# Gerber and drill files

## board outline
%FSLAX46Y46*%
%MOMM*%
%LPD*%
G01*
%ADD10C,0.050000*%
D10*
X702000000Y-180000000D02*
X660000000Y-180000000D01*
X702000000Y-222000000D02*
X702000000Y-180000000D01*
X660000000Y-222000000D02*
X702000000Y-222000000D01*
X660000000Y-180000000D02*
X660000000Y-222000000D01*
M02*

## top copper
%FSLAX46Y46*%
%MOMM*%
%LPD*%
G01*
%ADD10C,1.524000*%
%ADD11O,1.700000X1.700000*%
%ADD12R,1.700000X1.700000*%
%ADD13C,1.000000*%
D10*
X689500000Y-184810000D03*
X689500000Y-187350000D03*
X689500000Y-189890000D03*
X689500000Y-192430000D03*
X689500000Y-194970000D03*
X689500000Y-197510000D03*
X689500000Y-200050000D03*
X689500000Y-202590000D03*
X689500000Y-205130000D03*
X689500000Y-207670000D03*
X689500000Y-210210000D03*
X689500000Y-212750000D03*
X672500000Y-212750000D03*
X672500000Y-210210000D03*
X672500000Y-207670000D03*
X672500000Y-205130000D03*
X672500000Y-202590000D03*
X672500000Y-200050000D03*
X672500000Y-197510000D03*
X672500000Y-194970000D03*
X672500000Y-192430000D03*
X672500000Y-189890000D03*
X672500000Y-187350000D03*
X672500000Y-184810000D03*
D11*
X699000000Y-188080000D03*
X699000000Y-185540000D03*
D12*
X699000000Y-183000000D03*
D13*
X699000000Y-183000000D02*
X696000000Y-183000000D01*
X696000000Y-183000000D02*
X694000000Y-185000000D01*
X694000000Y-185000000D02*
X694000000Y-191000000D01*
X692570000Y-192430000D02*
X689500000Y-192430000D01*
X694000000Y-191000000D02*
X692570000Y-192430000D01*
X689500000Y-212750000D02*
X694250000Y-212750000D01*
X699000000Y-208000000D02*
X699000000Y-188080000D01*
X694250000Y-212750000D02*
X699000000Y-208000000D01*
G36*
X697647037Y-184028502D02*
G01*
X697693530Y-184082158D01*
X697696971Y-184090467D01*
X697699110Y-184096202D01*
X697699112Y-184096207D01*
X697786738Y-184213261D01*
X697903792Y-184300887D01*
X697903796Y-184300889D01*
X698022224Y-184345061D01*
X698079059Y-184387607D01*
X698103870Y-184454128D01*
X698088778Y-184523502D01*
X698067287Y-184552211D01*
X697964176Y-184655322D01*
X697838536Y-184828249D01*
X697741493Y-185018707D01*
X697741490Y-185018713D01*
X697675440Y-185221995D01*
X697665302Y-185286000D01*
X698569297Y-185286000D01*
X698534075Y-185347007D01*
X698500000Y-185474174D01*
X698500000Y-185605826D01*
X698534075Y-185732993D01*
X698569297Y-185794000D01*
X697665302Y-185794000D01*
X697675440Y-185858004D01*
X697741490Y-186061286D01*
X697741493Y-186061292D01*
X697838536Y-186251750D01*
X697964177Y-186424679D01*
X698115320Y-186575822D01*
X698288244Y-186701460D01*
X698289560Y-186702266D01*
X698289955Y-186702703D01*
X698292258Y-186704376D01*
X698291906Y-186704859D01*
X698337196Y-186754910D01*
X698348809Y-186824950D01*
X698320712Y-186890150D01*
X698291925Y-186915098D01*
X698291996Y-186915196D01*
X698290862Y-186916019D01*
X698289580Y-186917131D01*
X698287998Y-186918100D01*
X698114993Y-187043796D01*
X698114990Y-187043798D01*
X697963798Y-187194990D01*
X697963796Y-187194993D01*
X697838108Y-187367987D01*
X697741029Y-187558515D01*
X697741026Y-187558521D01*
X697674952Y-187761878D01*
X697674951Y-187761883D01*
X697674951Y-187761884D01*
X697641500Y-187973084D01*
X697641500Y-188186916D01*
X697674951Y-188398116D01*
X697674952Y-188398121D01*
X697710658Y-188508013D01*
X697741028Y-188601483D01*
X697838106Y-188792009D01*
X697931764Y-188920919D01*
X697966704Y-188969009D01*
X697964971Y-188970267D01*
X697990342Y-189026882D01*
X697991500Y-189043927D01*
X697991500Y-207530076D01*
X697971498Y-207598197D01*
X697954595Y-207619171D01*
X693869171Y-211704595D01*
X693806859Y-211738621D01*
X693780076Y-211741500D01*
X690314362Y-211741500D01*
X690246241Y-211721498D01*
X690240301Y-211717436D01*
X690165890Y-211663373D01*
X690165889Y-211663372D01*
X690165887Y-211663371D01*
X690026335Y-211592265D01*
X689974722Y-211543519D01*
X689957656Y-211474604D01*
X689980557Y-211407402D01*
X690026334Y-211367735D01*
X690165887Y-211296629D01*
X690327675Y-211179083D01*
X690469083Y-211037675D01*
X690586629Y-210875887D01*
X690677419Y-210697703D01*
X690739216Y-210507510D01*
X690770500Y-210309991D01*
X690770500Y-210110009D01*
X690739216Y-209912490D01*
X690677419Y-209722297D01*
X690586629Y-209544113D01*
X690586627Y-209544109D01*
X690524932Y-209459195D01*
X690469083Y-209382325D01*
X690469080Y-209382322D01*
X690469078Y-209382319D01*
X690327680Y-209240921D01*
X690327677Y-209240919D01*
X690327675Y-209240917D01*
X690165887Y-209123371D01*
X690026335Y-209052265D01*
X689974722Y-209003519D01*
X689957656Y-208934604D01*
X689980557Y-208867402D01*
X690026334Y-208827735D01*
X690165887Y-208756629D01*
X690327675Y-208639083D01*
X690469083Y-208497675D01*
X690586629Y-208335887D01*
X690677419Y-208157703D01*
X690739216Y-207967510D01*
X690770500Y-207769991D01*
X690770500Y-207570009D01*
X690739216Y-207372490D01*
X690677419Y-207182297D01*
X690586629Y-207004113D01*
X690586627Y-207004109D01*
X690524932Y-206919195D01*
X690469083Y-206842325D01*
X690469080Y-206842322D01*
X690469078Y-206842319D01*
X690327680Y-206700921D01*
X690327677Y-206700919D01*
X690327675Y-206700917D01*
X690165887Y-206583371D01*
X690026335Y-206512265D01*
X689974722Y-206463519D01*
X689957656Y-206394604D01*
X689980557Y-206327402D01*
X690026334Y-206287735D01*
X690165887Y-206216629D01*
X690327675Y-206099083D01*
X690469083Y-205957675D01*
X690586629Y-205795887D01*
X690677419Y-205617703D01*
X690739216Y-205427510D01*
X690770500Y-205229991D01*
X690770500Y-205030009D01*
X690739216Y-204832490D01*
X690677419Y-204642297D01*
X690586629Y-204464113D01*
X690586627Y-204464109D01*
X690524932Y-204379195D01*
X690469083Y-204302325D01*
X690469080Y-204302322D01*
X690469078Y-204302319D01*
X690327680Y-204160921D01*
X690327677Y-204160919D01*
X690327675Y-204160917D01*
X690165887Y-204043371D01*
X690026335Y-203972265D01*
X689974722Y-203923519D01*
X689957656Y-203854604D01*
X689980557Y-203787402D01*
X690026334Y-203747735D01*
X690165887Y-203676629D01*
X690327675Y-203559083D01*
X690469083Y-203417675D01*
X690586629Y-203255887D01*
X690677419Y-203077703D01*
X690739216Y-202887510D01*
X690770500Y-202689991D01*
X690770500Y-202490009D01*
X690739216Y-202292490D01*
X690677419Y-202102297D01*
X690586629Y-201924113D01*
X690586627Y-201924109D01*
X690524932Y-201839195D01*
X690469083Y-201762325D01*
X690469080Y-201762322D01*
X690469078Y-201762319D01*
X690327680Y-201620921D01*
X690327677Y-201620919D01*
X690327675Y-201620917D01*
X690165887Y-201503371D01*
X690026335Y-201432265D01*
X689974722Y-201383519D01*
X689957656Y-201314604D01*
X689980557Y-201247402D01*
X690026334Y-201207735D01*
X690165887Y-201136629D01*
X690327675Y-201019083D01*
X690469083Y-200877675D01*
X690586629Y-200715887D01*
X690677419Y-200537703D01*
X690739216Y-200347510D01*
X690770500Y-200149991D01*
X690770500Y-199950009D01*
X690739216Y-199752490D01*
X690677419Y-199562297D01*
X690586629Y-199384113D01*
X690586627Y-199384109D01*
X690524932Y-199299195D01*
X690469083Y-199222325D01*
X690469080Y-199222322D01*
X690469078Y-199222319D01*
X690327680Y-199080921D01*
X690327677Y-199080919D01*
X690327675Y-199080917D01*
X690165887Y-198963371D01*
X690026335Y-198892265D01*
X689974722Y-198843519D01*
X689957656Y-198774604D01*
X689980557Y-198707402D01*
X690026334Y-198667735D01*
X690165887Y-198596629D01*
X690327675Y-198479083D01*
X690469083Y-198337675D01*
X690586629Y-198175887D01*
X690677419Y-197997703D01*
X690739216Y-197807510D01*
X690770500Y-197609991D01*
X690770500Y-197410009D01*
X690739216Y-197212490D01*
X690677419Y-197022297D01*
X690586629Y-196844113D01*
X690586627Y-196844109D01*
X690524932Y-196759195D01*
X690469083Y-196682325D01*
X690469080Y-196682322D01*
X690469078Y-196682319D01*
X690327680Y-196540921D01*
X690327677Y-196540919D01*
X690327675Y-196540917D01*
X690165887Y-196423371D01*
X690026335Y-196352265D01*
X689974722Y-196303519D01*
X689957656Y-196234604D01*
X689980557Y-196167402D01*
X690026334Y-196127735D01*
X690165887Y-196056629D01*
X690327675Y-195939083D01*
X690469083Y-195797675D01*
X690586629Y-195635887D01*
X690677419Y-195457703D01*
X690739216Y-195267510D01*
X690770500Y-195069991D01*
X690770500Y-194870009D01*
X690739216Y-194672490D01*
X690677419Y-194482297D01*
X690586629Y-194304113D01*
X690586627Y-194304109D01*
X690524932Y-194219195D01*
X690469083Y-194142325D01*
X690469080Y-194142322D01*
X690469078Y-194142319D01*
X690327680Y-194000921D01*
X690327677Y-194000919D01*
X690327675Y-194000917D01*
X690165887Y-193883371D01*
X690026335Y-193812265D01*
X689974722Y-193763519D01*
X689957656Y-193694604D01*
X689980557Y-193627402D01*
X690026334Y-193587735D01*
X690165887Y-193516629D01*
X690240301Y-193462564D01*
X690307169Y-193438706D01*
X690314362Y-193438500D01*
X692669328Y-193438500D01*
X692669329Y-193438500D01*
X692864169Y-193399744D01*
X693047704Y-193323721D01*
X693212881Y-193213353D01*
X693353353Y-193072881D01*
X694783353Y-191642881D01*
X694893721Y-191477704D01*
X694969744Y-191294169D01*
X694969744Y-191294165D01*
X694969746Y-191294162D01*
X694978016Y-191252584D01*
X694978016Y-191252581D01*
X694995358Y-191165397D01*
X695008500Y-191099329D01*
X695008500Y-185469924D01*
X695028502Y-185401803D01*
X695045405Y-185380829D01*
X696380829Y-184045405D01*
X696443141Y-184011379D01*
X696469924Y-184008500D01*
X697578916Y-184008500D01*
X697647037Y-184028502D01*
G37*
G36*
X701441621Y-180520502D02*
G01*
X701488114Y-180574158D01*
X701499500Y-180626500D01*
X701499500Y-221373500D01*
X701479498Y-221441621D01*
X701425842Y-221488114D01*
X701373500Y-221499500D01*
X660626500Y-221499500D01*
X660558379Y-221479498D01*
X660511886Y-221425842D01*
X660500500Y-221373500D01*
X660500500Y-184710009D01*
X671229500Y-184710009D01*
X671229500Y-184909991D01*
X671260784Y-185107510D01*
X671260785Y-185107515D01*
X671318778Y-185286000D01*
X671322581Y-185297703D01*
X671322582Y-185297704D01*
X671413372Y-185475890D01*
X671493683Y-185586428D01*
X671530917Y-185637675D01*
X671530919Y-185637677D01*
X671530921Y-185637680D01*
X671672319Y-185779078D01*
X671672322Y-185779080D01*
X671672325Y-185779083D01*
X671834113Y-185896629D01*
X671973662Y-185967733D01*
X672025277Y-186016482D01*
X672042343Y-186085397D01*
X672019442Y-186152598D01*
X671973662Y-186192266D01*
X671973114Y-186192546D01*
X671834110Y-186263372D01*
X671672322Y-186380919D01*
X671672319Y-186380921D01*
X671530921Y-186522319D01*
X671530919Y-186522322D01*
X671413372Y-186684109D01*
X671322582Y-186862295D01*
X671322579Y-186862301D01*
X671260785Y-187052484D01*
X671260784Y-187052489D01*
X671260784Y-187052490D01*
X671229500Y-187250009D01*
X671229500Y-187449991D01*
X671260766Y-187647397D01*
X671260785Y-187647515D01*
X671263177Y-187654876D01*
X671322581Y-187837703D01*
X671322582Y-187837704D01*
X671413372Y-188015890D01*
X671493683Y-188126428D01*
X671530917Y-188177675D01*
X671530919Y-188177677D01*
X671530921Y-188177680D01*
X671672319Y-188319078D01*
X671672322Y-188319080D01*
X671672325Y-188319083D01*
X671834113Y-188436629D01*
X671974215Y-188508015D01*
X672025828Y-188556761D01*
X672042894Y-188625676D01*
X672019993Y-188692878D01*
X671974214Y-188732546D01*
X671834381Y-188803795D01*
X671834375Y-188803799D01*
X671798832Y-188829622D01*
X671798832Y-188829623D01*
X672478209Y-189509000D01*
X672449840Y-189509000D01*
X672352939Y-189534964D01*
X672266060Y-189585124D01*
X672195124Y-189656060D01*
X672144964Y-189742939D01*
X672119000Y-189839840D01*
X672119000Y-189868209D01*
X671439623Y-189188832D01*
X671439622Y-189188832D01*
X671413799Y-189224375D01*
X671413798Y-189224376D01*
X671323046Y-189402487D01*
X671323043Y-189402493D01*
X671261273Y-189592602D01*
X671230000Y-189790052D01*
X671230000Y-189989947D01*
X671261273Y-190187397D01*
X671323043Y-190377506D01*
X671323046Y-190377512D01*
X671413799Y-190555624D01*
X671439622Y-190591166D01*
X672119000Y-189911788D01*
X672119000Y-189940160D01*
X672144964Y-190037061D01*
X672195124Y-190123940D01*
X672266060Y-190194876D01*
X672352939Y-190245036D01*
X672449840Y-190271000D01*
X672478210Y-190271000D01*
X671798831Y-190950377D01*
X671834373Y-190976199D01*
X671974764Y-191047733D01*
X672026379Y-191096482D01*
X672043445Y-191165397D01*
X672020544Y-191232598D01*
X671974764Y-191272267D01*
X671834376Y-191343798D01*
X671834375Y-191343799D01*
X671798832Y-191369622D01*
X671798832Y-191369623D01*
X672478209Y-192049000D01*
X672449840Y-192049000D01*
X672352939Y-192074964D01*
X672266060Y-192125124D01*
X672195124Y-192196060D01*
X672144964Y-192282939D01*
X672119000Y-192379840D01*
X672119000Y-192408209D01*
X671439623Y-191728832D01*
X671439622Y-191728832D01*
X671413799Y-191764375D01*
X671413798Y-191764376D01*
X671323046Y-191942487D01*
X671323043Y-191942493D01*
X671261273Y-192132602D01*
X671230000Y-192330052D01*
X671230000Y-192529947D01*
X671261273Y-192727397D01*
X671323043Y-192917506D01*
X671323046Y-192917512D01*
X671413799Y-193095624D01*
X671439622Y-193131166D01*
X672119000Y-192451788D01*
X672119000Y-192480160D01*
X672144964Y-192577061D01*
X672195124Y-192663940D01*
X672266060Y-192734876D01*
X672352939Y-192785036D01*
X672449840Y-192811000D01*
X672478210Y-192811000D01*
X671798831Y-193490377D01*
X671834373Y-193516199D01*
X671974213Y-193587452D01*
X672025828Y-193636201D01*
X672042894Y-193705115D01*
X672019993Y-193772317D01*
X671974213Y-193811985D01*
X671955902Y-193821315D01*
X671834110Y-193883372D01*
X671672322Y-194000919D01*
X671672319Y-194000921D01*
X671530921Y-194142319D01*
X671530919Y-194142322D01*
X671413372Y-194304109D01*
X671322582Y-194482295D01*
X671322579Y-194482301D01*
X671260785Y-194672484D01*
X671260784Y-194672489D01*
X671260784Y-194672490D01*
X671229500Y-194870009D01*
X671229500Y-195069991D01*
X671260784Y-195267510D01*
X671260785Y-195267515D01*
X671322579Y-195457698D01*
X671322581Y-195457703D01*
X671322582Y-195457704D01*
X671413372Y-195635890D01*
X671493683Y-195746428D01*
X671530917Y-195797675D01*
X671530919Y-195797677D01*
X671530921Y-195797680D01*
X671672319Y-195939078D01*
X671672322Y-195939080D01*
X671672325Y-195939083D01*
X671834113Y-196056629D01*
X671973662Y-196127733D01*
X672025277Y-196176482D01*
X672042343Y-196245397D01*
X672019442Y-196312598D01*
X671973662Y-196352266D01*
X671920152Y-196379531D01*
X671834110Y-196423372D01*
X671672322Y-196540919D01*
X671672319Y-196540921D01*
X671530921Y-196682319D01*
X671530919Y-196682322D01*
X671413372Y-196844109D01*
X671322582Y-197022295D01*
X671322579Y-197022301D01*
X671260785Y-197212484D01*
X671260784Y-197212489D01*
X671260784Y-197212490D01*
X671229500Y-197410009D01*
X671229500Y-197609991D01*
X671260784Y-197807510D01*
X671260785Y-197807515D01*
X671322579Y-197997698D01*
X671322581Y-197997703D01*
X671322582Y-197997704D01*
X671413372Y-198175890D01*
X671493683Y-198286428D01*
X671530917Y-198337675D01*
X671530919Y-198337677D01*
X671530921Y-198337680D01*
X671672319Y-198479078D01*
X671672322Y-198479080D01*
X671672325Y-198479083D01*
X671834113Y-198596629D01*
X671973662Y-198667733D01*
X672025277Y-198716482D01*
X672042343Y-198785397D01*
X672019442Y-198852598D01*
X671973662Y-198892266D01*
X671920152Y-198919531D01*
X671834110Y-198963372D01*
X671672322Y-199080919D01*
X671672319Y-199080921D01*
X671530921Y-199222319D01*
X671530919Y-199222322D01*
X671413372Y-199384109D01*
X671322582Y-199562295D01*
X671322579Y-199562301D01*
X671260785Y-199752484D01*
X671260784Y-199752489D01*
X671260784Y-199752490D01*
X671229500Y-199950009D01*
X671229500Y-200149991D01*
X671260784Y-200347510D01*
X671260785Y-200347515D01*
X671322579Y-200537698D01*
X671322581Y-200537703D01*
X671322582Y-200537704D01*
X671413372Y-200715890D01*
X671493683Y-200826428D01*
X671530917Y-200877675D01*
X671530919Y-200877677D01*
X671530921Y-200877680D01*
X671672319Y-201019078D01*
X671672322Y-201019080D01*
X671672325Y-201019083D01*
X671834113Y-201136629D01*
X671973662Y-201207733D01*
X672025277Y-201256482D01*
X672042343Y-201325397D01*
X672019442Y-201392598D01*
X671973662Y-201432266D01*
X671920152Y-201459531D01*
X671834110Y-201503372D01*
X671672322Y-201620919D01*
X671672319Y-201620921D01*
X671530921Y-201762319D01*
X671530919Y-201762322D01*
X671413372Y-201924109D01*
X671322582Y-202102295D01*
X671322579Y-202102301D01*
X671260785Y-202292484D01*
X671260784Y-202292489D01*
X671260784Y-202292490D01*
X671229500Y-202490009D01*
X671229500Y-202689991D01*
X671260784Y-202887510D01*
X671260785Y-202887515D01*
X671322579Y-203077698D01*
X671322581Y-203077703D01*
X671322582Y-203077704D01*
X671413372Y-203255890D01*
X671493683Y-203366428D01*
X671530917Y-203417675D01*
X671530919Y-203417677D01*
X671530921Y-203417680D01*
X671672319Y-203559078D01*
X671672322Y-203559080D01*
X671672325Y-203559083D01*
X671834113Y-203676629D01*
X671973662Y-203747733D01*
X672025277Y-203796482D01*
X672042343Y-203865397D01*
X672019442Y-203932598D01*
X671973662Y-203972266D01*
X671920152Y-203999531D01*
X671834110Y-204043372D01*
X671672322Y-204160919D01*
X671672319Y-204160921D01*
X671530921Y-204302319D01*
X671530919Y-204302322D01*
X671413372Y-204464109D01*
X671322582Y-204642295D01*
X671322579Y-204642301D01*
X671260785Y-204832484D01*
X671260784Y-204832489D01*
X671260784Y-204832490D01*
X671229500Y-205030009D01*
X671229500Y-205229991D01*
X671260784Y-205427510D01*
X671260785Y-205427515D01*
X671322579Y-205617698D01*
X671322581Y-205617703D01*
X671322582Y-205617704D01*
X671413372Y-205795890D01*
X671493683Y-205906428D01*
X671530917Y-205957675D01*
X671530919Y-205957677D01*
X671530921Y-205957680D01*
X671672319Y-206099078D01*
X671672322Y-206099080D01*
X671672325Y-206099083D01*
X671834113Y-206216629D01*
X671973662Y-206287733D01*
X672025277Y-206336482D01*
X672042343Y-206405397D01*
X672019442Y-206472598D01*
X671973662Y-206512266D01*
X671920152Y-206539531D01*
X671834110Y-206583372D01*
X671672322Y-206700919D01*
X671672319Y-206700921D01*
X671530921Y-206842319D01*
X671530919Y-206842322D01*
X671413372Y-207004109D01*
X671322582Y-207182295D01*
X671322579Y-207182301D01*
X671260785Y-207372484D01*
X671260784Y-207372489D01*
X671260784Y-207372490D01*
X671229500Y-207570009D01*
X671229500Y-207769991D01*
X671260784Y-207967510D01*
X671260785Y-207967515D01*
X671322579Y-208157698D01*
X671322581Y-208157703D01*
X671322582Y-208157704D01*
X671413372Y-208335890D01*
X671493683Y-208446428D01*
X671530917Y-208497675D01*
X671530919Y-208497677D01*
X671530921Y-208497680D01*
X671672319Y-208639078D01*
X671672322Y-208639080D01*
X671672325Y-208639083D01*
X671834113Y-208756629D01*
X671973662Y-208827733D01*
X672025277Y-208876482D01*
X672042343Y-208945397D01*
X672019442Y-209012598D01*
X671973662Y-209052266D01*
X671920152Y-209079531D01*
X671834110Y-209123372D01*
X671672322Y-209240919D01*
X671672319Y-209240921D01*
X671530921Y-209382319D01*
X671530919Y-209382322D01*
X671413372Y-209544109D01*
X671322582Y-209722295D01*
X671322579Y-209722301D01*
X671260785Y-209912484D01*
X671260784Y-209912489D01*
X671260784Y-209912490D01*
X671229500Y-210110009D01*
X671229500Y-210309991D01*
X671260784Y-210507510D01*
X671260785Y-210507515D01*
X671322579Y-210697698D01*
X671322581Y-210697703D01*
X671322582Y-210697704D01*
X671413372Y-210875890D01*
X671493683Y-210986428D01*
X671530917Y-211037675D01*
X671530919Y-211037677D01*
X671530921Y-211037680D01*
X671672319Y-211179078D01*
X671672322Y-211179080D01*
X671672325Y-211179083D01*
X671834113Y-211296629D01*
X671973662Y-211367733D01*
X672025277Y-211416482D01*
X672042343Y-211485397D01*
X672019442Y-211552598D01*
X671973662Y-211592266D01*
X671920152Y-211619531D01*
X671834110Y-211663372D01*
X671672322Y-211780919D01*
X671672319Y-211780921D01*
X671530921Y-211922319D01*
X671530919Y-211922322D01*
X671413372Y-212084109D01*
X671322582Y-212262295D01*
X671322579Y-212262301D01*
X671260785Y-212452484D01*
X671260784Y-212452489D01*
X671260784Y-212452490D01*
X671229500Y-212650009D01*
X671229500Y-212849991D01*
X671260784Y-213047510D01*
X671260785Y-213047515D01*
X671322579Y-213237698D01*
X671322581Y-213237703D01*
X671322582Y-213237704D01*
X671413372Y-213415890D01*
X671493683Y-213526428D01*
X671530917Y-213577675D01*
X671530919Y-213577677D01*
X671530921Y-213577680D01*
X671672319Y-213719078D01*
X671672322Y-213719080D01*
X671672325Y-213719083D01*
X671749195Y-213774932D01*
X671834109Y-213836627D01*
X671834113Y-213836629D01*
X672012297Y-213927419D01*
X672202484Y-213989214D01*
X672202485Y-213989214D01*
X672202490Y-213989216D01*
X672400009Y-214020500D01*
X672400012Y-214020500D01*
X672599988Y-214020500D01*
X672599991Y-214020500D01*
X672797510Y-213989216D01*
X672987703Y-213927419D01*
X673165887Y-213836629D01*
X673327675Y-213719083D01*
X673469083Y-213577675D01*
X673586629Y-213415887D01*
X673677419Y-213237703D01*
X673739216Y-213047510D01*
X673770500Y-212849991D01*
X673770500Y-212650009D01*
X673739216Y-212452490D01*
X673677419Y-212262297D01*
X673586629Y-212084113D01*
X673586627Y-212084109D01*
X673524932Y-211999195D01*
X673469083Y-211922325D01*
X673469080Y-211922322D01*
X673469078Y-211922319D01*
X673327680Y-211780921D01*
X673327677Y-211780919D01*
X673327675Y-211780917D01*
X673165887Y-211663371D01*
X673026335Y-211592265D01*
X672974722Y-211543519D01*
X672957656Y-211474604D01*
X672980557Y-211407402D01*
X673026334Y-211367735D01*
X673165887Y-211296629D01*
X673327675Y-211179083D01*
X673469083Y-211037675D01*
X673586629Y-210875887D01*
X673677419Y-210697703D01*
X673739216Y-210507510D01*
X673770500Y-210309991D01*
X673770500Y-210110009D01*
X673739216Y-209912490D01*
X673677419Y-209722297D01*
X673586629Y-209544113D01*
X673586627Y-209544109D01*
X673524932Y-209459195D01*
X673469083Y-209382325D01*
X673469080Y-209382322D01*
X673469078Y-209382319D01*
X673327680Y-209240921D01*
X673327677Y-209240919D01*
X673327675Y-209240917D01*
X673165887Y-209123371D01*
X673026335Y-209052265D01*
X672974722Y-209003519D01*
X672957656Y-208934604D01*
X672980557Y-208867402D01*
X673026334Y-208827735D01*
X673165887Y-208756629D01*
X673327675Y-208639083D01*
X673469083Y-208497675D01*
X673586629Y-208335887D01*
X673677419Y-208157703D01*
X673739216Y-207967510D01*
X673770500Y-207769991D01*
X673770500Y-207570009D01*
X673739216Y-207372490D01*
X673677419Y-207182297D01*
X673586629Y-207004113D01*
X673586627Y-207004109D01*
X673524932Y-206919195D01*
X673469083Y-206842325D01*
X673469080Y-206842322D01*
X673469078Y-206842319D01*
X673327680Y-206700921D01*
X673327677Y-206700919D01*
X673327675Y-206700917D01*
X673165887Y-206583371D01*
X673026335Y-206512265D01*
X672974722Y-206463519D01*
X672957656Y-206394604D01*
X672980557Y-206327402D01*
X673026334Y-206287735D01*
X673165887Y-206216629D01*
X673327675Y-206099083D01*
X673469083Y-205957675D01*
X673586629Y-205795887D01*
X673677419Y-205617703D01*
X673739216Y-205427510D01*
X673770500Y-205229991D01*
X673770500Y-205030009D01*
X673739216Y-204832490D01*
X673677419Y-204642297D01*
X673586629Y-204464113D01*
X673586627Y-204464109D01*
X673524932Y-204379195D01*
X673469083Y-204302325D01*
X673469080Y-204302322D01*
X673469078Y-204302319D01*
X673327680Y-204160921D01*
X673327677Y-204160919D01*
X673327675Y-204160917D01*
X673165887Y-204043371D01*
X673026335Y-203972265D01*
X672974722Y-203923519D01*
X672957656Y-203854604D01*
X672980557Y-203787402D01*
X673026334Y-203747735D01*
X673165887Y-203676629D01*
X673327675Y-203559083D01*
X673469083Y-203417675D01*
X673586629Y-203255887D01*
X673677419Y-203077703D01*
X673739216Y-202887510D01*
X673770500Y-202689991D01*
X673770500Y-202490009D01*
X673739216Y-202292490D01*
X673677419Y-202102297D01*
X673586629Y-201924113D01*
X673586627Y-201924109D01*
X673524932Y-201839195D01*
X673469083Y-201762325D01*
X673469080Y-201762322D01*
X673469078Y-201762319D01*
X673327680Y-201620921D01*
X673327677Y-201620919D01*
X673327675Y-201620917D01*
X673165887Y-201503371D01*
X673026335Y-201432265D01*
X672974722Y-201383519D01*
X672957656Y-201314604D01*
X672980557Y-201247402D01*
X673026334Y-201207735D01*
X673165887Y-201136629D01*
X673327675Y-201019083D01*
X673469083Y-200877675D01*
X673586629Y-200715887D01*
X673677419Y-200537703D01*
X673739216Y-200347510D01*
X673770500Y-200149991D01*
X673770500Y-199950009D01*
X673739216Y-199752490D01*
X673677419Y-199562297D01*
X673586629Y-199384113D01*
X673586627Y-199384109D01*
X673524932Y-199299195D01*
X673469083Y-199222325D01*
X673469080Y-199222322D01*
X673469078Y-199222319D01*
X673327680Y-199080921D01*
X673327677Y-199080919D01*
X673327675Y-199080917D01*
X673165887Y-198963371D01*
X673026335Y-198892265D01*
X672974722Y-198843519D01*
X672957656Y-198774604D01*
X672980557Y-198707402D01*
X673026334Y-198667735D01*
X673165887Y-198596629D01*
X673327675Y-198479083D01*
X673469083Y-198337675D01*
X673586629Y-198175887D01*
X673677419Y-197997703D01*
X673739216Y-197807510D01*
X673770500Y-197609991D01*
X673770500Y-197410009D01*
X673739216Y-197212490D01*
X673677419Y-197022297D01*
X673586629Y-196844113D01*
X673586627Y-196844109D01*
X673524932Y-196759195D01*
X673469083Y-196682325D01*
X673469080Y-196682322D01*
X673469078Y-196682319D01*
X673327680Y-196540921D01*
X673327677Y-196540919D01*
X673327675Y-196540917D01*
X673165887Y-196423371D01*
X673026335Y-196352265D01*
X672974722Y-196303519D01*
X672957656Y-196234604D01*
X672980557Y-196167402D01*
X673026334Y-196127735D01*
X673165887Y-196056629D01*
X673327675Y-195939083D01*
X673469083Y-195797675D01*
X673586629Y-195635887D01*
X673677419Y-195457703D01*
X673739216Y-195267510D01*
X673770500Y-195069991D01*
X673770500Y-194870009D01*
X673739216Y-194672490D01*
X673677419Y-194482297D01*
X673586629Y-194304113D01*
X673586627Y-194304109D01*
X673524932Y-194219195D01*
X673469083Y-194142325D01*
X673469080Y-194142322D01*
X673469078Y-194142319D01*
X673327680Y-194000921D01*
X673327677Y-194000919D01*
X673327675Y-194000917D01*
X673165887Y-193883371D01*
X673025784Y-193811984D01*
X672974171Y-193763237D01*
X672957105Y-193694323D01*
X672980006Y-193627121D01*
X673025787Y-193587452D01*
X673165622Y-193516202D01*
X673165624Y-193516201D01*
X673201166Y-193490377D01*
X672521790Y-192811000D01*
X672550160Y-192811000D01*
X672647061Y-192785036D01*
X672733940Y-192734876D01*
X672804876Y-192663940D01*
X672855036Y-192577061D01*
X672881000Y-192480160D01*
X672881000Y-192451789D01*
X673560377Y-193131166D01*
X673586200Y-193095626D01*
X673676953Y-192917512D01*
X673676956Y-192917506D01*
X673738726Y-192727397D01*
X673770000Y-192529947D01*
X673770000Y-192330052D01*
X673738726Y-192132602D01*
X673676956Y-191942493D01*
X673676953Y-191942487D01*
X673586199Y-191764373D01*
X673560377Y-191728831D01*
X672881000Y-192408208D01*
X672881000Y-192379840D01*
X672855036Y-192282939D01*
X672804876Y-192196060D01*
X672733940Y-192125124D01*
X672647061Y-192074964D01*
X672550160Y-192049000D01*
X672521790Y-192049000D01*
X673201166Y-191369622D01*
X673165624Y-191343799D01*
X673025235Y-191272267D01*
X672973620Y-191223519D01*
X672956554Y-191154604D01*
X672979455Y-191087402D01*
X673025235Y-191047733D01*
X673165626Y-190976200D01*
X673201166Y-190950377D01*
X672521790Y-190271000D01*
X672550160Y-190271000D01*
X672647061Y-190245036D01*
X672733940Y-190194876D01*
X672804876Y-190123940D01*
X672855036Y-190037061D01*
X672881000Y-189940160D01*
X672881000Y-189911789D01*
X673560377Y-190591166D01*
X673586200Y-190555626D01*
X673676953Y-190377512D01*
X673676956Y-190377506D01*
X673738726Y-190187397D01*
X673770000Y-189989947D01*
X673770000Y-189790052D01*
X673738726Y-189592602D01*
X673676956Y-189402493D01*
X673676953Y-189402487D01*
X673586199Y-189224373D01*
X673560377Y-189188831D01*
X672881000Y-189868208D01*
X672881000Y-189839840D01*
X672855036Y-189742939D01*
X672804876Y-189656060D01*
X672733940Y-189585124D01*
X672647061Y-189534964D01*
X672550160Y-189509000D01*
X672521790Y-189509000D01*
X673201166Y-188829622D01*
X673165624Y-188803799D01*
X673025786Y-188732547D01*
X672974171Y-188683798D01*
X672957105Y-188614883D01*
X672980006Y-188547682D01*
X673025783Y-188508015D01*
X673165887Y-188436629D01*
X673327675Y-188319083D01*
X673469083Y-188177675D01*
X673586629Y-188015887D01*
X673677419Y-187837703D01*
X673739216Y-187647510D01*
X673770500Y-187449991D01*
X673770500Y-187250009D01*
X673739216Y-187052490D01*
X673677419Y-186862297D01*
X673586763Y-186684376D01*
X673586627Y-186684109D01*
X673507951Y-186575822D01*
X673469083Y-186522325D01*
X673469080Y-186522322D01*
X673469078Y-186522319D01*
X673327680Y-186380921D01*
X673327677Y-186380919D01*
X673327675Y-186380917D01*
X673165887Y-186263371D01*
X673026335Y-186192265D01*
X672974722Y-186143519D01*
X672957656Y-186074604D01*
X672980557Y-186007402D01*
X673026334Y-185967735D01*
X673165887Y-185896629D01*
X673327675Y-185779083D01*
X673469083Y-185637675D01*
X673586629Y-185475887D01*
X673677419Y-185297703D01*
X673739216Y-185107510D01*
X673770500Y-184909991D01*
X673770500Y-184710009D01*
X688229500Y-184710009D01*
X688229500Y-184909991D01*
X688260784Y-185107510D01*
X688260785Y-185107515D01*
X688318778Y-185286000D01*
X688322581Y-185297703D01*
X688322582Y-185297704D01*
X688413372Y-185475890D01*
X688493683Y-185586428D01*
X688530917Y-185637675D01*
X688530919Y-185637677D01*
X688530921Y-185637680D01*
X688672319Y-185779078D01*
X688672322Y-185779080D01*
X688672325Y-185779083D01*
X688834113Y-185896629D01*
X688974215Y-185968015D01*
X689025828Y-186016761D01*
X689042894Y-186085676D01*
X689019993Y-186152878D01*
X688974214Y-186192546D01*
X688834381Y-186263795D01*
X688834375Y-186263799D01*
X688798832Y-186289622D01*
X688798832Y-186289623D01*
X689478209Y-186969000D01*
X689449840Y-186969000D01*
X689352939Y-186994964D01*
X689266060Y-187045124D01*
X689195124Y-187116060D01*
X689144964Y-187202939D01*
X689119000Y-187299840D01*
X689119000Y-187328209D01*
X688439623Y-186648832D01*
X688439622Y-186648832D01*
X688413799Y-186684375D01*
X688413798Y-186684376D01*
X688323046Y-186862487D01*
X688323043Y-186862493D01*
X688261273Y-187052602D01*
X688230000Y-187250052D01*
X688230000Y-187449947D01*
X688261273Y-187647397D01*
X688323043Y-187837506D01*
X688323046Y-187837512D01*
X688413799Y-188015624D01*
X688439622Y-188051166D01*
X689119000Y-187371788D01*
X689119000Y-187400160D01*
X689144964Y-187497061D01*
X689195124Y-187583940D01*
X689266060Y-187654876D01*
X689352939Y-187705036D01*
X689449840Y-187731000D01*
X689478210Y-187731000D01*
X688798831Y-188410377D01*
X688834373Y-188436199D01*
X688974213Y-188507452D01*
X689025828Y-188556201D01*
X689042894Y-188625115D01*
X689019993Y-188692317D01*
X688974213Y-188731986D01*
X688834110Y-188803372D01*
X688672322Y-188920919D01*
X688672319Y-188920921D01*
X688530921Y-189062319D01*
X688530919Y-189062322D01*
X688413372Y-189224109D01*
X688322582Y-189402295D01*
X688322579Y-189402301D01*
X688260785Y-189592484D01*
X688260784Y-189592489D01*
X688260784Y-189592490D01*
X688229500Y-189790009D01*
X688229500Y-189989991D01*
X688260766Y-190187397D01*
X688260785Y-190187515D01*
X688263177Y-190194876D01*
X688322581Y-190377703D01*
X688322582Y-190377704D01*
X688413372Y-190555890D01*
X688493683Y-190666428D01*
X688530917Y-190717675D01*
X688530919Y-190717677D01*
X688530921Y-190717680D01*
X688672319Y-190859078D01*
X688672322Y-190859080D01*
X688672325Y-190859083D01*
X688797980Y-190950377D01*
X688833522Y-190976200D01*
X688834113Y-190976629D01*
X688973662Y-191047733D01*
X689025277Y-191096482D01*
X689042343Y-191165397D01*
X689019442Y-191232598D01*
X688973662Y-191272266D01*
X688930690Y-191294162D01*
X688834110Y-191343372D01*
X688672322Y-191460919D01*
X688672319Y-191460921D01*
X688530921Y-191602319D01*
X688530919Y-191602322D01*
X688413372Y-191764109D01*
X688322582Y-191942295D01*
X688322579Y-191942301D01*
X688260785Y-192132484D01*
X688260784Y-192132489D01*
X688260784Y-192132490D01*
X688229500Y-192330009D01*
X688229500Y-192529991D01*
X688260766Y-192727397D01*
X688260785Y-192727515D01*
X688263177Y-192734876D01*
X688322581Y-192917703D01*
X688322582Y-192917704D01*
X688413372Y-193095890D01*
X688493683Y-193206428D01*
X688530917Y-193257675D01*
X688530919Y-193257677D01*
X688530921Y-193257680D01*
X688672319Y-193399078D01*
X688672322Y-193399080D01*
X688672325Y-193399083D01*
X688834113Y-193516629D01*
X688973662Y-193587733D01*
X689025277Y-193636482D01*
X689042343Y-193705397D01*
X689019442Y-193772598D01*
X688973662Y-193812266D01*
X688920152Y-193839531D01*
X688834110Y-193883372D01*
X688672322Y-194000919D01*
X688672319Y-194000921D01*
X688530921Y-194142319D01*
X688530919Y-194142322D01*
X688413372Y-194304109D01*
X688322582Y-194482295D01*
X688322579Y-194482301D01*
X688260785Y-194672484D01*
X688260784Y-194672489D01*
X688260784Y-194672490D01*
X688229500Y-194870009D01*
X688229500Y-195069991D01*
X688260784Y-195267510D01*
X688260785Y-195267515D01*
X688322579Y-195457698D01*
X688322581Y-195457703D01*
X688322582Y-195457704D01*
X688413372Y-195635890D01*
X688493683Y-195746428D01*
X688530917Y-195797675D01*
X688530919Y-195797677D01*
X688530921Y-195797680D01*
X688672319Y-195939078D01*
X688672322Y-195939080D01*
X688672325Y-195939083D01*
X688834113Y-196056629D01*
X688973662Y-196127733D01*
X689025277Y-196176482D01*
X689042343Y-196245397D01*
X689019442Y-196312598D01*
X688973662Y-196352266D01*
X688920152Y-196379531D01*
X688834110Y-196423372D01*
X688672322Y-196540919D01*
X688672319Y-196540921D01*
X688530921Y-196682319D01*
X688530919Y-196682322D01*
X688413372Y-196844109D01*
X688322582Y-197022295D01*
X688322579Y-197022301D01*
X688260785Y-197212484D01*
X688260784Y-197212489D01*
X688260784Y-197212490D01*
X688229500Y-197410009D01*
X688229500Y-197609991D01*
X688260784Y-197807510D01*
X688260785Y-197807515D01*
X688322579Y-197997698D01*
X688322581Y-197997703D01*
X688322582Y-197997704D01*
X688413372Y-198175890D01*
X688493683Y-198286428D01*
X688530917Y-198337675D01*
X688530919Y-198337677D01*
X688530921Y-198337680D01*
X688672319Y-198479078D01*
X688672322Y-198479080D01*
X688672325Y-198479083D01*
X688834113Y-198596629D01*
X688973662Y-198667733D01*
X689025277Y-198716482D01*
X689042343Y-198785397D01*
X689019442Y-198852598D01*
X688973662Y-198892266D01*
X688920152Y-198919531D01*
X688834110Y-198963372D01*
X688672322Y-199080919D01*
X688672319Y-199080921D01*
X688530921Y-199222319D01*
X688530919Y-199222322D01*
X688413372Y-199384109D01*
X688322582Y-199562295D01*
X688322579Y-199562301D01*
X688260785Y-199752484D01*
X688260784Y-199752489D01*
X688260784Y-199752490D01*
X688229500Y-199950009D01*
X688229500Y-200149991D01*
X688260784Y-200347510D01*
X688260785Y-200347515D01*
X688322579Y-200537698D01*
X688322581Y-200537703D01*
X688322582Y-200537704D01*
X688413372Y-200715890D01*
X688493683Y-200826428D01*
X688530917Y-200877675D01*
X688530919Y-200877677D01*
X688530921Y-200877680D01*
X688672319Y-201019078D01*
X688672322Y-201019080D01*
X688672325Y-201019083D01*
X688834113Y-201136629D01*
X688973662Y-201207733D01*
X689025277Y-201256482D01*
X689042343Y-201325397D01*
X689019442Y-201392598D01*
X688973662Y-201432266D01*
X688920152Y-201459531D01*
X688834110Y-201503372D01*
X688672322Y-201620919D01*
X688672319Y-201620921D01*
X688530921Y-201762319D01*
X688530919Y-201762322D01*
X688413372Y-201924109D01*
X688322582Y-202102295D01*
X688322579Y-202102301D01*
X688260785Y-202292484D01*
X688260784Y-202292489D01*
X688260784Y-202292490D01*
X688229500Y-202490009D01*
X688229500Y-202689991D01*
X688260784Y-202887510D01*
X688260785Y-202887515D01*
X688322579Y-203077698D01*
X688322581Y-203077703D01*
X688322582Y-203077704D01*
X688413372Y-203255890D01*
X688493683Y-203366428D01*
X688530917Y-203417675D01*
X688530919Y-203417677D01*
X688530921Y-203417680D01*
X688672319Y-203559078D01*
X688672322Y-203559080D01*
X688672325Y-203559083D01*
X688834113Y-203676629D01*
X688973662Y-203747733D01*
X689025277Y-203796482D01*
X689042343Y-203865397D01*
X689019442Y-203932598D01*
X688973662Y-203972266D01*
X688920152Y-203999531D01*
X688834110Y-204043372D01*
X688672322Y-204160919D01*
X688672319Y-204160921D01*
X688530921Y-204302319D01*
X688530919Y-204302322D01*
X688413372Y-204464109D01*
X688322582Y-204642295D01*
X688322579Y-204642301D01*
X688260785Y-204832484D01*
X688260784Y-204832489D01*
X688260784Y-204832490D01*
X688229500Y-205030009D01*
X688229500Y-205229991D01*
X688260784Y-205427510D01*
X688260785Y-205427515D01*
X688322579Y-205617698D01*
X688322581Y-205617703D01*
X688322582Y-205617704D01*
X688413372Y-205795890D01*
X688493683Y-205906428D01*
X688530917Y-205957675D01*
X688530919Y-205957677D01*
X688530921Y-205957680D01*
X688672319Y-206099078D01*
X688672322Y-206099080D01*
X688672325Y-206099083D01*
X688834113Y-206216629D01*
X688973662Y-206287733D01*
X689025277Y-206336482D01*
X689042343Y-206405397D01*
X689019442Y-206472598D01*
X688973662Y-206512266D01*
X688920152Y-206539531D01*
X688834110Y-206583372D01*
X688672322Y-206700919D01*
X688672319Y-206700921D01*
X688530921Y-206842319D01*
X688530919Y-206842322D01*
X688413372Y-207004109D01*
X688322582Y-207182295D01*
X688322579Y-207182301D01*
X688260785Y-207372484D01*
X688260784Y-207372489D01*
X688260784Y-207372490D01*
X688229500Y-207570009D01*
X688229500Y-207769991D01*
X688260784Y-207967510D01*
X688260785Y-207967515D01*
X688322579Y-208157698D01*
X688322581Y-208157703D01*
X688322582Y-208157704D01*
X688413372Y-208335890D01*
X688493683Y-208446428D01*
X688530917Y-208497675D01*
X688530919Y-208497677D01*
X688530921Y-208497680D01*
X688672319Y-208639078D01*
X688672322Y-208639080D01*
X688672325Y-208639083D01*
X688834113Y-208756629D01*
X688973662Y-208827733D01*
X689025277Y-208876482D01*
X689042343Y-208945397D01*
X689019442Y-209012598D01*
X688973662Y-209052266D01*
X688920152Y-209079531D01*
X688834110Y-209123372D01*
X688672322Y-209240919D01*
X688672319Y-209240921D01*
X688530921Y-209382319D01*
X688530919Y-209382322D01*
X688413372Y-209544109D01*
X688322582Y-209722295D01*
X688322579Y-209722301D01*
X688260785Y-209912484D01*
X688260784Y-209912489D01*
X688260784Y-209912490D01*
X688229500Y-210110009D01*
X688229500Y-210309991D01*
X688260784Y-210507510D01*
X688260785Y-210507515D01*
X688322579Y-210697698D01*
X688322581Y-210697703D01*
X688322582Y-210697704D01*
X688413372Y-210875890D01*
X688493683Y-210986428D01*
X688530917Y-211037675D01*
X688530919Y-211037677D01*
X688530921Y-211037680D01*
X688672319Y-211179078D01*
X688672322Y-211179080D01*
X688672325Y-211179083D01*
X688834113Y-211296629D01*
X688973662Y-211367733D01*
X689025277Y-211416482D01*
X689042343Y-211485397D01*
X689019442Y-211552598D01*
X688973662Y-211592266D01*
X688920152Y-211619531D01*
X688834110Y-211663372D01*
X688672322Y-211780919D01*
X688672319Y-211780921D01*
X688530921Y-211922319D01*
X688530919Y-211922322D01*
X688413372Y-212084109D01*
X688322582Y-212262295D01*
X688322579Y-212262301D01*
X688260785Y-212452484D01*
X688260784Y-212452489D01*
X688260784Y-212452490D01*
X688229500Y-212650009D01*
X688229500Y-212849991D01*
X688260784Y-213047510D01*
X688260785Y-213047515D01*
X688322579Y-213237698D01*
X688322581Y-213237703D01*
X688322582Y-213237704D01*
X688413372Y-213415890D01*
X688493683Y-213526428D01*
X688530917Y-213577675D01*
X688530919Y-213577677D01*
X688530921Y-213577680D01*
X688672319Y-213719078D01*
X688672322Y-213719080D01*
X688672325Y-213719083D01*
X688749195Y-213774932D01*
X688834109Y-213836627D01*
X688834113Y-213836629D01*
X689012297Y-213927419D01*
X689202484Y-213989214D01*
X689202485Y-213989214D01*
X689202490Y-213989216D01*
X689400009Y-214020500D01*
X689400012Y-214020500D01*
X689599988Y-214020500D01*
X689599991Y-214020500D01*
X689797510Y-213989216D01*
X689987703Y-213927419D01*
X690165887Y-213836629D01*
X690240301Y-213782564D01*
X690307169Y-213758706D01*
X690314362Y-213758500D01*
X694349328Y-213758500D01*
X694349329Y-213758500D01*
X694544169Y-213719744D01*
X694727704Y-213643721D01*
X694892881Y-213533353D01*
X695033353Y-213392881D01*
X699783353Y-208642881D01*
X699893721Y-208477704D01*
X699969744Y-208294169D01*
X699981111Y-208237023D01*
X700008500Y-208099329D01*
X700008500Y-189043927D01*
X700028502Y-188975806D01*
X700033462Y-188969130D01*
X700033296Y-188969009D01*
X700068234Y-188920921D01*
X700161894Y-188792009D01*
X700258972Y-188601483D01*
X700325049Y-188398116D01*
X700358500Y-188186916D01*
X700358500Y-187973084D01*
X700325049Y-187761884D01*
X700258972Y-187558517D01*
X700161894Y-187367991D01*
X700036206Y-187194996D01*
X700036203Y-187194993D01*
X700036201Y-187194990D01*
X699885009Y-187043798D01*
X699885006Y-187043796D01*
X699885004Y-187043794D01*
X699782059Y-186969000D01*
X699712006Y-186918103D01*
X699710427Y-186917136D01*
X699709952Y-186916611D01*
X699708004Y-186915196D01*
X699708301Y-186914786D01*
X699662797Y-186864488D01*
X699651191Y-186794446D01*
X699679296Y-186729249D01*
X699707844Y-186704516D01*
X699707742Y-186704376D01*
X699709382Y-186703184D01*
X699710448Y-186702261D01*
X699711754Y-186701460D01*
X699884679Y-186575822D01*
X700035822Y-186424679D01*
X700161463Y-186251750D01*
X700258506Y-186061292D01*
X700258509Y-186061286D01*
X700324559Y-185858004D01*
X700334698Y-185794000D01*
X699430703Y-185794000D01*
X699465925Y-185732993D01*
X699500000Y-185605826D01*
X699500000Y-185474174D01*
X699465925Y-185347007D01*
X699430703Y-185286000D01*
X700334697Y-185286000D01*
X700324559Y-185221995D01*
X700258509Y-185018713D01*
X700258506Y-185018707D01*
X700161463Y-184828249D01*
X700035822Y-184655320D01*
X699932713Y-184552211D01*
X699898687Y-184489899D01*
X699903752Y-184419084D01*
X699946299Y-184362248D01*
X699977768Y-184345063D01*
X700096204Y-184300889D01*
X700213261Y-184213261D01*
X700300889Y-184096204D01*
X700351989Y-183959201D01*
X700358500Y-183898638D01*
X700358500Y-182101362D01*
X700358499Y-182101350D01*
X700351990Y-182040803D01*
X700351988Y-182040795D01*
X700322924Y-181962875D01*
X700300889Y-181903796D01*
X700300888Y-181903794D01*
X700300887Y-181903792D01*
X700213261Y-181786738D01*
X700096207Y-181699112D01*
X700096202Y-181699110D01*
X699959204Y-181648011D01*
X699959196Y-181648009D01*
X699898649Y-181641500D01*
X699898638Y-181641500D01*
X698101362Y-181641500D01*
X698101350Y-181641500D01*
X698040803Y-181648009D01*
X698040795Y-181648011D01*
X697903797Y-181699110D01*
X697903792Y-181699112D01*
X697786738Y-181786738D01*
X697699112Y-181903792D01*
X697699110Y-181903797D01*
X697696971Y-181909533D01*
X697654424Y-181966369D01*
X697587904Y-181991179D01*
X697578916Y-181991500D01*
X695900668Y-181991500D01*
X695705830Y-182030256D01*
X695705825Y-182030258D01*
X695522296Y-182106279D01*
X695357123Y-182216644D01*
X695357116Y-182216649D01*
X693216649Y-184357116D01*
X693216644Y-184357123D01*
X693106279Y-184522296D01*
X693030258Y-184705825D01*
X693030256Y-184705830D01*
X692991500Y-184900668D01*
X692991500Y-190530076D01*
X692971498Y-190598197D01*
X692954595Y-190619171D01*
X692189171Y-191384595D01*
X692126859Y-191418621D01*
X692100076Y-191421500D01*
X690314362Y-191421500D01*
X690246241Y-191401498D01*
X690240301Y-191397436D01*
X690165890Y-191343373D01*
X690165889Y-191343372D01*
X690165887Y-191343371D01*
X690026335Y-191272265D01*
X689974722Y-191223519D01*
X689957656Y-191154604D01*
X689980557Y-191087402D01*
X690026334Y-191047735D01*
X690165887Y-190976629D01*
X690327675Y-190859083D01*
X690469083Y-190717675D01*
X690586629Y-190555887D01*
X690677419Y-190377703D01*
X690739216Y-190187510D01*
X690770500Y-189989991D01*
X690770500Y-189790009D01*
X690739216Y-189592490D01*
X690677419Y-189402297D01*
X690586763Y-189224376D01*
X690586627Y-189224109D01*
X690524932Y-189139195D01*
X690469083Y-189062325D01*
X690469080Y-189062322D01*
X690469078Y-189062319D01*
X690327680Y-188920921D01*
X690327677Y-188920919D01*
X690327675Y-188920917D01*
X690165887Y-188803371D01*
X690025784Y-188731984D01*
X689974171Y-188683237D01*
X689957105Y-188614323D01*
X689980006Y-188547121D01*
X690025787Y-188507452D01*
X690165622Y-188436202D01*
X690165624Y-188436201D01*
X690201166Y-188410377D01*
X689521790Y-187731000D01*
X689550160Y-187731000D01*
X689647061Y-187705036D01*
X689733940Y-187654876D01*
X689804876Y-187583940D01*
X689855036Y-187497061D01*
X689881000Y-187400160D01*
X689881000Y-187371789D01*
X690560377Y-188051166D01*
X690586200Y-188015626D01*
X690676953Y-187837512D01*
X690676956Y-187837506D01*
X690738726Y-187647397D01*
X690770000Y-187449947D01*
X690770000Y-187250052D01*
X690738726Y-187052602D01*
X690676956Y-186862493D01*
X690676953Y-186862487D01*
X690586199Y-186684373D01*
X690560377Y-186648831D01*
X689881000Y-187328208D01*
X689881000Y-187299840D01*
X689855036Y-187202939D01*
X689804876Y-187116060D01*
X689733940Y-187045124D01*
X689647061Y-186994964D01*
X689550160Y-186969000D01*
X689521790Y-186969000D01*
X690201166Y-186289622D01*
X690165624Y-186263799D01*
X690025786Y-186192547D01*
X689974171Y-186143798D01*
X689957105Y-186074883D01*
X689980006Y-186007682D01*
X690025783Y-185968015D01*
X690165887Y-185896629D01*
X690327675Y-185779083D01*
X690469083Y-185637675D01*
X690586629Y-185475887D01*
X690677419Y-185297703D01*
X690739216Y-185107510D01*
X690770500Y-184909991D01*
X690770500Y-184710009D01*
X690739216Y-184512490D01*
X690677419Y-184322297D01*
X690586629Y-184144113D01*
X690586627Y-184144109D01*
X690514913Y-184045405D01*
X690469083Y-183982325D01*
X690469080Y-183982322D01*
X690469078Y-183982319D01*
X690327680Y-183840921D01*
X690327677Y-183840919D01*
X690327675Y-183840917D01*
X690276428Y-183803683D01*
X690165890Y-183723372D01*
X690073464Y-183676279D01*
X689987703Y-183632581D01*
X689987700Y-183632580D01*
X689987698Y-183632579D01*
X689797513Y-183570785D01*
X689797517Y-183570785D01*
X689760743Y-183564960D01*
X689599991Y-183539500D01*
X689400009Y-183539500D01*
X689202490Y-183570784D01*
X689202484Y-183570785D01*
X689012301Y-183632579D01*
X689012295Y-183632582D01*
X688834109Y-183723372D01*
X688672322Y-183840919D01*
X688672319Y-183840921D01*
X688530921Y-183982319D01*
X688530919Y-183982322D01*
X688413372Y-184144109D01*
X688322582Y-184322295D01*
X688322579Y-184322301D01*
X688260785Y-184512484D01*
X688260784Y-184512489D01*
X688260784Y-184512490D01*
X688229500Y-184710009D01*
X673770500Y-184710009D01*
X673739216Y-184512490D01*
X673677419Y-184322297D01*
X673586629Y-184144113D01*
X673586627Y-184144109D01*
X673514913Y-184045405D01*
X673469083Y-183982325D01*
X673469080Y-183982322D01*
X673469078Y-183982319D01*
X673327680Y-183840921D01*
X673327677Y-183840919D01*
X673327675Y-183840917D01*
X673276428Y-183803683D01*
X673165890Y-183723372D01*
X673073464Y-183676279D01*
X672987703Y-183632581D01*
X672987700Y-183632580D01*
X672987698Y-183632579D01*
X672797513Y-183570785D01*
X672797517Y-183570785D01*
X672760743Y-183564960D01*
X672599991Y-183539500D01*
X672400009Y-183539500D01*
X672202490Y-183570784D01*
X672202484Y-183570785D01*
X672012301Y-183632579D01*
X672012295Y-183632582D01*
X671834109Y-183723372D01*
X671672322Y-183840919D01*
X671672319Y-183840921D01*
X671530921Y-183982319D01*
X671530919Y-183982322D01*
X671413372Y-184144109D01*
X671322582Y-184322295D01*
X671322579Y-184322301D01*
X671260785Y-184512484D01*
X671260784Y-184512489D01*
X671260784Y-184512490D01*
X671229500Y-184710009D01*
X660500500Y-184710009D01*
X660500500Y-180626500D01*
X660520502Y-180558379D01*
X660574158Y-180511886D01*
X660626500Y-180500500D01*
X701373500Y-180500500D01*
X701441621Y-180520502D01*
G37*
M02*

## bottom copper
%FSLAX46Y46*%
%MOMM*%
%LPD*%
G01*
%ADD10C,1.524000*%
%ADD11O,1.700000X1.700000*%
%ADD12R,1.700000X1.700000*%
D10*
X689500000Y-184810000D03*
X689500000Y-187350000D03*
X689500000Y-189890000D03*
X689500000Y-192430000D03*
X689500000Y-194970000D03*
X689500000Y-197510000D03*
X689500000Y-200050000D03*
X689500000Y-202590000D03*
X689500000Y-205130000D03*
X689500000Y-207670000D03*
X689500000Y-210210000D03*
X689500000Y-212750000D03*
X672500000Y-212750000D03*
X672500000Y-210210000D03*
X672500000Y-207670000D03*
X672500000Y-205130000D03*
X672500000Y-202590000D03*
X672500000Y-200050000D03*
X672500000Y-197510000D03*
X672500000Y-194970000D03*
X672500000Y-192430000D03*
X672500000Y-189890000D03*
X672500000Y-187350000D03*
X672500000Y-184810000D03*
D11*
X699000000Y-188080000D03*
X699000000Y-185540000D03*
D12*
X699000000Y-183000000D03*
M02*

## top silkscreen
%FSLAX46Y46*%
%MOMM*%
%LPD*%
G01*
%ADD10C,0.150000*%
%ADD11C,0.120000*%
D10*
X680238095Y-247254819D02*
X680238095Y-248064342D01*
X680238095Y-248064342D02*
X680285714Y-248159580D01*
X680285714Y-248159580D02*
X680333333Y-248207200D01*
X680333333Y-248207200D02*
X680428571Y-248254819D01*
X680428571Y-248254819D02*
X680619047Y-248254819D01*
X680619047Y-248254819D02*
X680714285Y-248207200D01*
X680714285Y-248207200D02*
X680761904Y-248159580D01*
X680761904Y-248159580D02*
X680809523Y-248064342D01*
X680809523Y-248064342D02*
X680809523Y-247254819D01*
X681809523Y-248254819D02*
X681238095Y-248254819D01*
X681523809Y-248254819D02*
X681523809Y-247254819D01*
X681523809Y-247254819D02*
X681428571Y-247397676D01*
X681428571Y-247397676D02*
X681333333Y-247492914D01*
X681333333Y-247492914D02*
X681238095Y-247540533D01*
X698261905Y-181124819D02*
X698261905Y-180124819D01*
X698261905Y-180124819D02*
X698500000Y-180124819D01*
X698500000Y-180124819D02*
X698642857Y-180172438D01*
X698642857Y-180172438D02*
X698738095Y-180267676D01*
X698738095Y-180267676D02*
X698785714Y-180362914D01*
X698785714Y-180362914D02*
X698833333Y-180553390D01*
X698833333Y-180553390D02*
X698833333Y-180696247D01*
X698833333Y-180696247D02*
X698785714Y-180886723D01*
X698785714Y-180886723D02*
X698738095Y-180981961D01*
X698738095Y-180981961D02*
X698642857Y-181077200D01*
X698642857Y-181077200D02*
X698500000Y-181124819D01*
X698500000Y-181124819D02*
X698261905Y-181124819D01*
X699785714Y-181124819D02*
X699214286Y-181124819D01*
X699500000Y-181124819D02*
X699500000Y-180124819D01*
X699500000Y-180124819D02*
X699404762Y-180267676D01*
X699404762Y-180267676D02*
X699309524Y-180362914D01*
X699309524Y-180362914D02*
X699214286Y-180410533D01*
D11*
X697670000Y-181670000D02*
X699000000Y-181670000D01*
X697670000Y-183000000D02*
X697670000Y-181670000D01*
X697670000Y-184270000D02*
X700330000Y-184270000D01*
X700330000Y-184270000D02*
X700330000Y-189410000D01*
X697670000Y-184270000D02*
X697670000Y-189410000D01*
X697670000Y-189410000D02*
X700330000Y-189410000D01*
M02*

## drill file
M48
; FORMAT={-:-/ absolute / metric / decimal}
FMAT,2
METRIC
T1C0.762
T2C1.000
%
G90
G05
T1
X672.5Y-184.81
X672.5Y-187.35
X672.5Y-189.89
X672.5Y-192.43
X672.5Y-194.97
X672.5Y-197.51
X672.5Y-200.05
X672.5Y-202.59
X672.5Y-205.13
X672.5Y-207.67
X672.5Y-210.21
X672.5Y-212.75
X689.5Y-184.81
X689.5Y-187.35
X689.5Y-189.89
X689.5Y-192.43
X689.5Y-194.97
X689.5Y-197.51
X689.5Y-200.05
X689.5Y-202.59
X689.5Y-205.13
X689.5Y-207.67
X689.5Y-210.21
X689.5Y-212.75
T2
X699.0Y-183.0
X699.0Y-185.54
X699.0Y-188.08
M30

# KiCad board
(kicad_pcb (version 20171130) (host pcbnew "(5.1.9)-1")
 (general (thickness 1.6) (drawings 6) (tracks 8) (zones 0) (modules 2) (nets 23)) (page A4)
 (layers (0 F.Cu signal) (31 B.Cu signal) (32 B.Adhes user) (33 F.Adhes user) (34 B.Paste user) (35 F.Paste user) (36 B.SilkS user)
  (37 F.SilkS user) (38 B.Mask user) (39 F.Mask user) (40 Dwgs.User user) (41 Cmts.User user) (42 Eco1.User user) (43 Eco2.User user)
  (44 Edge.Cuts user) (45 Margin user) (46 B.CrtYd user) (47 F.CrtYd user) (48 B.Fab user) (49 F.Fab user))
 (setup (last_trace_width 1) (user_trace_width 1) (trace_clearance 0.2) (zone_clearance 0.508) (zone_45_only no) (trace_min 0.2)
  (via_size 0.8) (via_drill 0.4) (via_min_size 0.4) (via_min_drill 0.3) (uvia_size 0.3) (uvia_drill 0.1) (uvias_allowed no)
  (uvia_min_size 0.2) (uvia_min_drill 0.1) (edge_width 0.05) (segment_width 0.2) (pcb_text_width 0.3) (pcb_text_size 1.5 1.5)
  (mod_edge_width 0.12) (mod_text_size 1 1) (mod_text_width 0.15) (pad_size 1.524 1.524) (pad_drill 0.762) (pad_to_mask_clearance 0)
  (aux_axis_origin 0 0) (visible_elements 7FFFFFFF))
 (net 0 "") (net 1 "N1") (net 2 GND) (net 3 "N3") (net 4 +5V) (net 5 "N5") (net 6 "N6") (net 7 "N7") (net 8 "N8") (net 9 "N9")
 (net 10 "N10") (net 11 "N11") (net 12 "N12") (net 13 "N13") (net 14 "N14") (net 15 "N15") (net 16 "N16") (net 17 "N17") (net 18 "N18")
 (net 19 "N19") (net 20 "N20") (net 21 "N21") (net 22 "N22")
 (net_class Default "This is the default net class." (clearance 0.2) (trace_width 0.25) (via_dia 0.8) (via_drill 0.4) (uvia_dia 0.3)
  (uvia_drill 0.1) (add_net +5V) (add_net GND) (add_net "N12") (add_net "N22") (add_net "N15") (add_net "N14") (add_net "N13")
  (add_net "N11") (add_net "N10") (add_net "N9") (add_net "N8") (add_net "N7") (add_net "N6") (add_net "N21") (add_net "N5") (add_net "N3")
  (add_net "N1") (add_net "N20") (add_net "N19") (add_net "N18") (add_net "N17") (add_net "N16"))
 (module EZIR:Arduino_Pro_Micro (layer F.Cu) (at 681 197)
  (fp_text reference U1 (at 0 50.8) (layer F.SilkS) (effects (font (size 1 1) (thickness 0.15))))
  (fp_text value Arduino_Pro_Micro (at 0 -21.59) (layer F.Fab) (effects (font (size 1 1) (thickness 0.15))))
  (pad 24 thru_hole circle (at 8.5 -12.19) (size 1.524 1.524) (drill 0.762) (layers *.Cu *.Mask) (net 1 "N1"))
  (pad 23 thru_hole circle (at 8.5 -9.65) (size 1.524 1.524) (drill 0.762) (layers *.Cu *.Mask) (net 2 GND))
  (pad 22 thru_hole circle (at 8.5 -7.11) (size 1.524 1.524) (drill 0.762) (layers *.Cu *.Mask) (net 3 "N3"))
  (pad 21 thru_hole circle (at 8.5 -4.57) (size 1.524 1.524) (drill 0.762) (layers *.Cu *.Mask) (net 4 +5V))
  (pad 20 thru_hole circle (at 8.5 -2.03) (size 1.524 1.524) (drill 0.762) (layers *.Cu *.Mask) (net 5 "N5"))
  (pad 19 thru_hole circle (at 8.5 0.51) (size 1.524 1.524) (drill 0.762) (layers *.Cu *.Mask) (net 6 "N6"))
  (pad 18 thru_hole circle (at 8.5 3.05) (size 1.524 1.524) (drill 0.762) (layers *.Cu *.Mask) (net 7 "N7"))
  (pad 17 thru_hole circle (at 8.5 5.59) (size 1.524 1.524) (drill 0.762) (layers *.Cu *.Mask) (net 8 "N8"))
  (pad 16 thru_hole circle (at 8.5 8.13) (size 1.524 1.524) (drill 0.762) (layers *.Cu *.Mask) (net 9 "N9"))
  (pad 15 thru_hole circle (at 8.5 10.67) (size 1.524 1.524) (drill 0.762) (layers *.Cu *.Mask) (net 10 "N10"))
  (pad 14 thru_hole circle (at 8.5 13.21) (size 1.524 1.524) (drill 0.762) (layers *.Cu *.Mask) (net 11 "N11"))
  (pad 13 thru_hole circle (at 8.5 15.75) (size 1.524 1.524) (drill 0.762) (layers *.Cu *.Mask) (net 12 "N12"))
  (pad 12 thru_hole circle (at -8.5 15.75) (size 1.524 1.524) (drill 0.762) (layers *.Cu *.Mask) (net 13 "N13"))
  (pad 11 thru_hole circle (at -8.5 13.21) (size 1.524 1.524) (drill 0.762) (layers *.Cu *.Mask) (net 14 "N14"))
  (pad 10 thru_hole circle (at -8.5 10.67) (size 1.524 1.524) (drill 0.762) (layers *.Cu *.Mask) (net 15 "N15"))
  (pad 9 thru_hole circle (at -8.5 8.13) (size 1.524 1.524) (drill 0.762) (layers *.Cu *.Mask) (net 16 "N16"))
  (pad 8 thru_hole circle (at -8.5 5.59) (size 1.524 1.524) (drill 0.762) (layers *.Cu *.Mask) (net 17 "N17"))
  (pad 7 thru_hole circle (at -8.5 3.05) (size 1.524 1.524) (drill 0.762) (layers *.Cu *.Mask) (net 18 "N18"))
  (pad 6 thru_hole circle (at -8.5 0.51) (size 1.524 1.524) (drill 0.762) (layers *.Cu *.Mask) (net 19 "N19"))
  (pad 5 thru_hole circle (at -8.5 -2.03) (size 1.524 1.524) (drill 0.762) (layers *.Cu *.Mask) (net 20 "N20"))
  (pad 4 thru_hole circle (at -8.5 -4.57) (size 1.524 1.524) (drill 0.762) (layers *.Cu *.Mask) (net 2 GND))
  (pad 3 thru_hole circle (at -8.5 -7.11) (size 1.524 1.524) (drill 0.762) (layers *.Cu *.Mask) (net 2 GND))
  (pad 2 thru_hole circle (at -8.5 -9.65) (size 1.524 1.524) (drill 0.762) (layers *.Cu *.Mask) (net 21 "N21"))
  (pad 1 thru_hole circle (at -8.5 -12.19) (size 1.524 1.524) (drill 0.762) (layers *.Cu *.Mask) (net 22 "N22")))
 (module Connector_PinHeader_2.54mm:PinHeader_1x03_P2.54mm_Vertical (layer F.Cu) (at 699 183)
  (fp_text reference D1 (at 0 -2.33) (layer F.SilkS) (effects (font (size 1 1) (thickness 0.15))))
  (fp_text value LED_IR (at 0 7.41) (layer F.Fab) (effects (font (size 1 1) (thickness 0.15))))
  (fp_line (start -1.33 -1.33) (end 0 -1.33) (layer F.SilkS) (width 0.12))
  (fp_line (start -1.33 0) (end -1.33 -1.33) (layer F.SilkS) (width 0.12))
  (fp_line (start -1.33 1.27) (end 1.33 1.27) (layer F.SilkS) (width 0.12))
  (fp_line (start 1.33 1.27) (end 1.33 6.41) (layer F.SilkS) (width 0.12))
  (fp_line (start -1.33 1.27) (end -1.33 6.41) (layer F.SilkS) (width 0.12))
  (fp_line (start -1.33 6.41) (end 1.33 6.41) (layer F.SilkS) (width 0.12))
  (pad 3 thru_hole oval (at 0 5.08) (size 1.7 1.7) (drill 1) (layers *.Cu *.Mask) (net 12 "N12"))
  (pad 2 thru_hole oval (at 0 2.54) (size 1.7 1.7) (drill 1) (layers *.Cu *.Mask) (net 2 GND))
  (pad 1 thru_hole rect (at 0 0) (size 1.7 1.7) (drill 1) (layers *.Cu *.Mask) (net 4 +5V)))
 (gr_line (start 702 180) (end 660 180) (layer Edge.Cuts) (width 0.05))
 (gr_line (start 702 222) (end 702 180) (layer Edge.Cuts) (width 0.05))
 (gr_line (start 660 222) (end 702 222) (layer Edge.Cuts) (width 0.05))
 (gr_line (start 660 180) (end 660 222) (layer Edge.Cuts) (width 0.05))
 (segment (start 699 183) (end 696 183) (width 1) (layer F.Cu) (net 4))
 (segment (start 696 183) (end 694 185) (width 1) (layer F.Cu) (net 4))
 (segment (start 694 185) (end 694 191) (width 1) (layer F.Cu) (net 4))
 (segment (start 692.57 192.43) (end 689.5 192.43) (width 1) (layer F.Cu) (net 4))
 (segment (start 694 191) (end 692.57 192.43) (width 1) (layer F.Cu) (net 4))
 (segment (start 689.5 212.75) (end 694.25 212.75) (width 1) (layer F.Cu) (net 12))
 (segment (start 699 208) (end 699 188.08) (width 1) (layer F.Cu) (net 12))
 (segment (start 694.25 212.75) (end 699 208) (width 1) (layer F.Cu) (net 12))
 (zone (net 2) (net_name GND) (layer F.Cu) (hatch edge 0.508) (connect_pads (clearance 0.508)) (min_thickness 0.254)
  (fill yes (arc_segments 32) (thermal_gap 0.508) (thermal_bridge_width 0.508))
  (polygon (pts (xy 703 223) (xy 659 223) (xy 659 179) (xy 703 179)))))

